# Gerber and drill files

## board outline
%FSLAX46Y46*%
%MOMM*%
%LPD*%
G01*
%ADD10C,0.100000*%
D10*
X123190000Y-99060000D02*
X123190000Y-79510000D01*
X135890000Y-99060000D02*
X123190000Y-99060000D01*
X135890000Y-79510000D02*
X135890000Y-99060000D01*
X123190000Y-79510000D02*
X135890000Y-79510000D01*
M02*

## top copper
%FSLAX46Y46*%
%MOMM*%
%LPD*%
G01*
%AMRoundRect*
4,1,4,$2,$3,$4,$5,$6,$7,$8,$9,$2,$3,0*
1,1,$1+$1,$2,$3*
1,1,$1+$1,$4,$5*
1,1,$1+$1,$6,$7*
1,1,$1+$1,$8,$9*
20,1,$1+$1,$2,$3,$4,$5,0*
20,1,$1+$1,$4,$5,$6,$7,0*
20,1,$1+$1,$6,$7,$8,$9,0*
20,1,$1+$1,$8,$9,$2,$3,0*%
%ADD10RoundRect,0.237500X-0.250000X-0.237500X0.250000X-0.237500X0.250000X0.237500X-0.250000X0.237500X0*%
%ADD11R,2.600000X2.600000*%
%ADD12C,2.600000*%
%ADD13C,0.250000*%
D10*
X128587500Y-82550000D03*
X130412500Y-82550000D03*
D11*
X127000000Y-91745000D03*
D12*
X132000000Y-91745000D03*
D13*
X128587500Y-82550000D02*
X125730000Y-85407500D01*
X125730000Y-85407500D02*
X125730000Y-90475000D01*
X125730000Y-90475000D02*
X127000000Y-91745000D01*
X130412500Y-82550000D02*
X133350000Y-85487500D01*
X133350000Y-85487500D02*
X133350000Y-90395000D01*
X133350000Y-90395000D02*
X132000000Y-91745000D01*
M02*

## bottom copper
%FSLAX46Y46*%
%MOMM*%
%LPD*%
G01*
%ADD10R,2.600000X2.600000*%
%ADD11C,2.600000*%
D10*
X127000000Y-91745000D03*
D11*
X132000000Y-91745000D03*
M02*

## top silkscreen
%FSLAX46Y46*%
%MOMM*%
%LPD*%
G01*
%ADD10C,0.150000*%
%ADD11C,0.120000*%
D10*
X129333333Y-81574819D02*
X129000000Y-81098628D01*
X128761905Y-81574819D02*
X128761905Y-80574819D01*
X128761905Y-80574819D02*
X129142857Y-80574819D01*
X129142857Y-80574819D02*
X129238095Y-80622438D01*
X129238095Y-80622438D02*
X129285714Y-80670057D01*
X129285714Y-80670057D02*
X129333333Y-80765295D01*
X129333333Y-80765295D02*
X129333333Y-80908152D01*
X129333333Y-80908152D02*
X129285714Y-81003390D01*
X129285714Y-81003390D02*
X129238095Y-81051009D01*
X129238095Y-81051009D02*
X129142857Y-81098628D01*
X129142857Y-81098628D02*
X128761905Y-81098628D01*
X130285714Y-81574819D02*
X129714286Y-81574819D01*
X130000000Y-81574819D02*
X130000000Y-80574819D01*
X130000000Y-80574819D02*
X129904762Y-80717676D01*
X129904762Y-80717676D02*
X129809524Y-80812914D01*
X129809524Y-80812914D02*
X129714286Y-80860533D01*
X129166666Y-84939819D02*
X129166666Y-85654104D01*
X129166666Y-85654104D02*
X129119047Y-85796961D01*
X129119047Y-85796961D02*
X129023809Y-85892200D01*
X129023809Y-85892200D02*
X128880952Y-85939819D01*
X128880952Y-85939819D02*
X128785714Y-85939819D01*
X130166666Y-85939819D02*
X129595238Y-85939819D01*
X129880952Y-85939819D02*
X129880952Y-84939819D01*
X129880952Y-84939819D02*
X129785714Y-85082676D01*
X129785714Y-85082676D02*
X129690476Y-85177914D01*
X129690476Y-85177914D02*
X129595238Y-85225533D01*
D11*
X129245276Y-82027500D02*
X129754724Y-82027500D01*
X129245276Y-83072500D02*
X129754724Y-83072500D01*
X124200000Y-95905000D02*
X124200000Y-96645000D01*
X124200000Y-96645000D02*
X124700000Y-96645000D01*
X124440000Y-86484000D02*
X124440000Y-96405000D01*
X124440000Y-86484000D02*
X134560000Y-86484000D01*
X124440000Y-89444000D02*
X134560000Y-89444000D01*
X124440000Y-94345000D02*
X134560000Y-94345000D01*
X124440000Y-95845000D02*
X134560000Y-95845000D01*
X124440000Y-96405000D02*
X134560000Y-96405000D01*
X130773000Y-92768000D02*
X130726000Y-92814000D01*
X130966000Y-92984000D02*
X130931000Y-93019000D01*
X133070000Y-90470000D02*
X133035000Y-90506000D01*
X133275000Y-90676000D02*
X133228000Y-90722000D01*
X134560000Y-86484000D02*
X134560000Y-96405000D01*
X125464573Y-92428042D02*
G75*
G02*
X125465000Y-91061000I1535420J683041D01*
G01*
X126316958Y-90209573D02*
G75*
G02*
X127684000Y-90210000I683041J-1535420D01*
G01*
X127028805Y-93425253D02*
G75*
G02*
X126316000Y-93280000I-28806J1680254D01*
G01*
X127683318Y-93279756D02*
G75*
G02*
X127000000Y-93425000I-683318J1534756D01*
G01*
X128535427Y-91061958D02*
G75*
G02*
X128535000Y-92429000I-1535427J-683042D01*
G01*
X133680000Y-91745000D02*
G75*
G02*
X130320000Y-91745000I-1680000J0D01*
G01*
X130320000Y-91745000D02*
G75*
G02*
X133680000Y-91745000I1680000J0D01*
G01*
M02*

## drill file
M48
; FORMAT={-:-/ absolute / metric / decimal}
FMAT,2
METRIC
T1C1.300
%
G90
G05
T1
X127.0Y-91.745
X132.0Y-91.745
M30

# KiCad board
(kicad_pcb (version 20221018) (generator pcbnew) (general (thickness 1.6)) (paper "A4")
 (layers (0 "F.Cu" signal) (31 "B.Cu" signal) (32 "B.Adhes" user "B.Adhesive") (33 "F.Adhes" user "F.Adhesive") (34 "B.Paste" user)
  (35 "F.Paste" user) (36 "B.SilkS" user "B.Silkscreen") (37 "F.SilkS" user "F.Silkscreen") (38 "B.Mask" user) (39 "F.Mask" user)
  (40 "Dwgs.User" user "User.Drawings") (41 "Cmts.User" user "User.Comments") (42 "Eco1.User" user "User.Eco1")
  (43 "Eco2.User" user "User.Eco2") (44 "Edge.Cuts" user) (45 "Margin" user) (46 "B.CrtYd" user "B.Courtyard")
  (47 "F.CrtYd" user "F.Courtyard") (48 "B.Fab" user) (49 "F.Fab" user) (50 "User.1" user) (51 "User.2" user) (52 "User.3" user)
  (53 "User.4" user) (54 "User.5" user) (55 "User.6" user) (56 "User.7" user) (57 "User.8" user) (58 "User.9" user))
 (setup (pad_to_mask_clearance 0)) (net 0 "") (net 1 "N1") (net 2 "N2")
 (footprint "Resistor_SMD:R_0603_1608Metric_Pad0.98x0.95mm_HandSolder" (layer "F.Cu") (at 129.5 82.55)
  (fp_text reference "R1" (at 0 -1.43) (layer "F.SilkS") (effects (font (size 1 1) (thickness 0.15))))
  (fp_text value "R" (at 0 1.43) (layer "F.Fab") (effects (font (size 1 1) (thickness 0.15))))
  (fp_line (start -0.254724 -0.5225) (end 0.254724 -0.5225) (stroke (width 0.12) (type solid)) (layer "F.SilkS"))
  (fp_line (start -0.254724 0.5225) (end 0.254724 0.5225) (stroke (width 0.12) (type solid)) (layer "F.SilkS"))
  (pad "1" smd roundrect (at -0.9125 0) (size 0.975 0.95) (layers "F.Cu" "F.Paste" "F.Mask") (roundrect_rratio 0.25) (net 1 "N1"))
  (pad "2" smd roundrect (at 0.9125 0) (size 0.975 0.95) (layers "F.Cu" "F.Paste" "F.Mask") (roundrect_rratio 0.25) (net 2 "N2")))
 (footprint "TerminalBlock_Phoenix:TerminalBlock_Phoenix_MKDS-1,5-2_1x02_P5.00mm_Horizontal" (layer "F.Cu") (at 127 91.745)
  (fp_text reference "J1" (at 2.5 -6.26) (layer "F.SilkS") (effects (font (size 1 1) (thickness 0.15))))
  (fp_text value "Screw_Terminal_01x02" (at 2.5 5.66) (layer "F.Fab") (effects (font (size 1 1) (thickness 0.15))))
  (fp_line (start -2.8 4.16) (end -2.8 4.9) (stroke (width 0.12) (type solid)) (layer "F.SilkS"))
  (fp_line (start -2.8 4.9) (end -2.3 4.9) (stroke (width 0.12) (type solid)) (layer "F.SilkS"))
  (fp_line (start -2.56 -5.261) (end -2.56 4.66) (stroke (width 0.12) (type solid)) (layer "F.SilkS"))
  (fp_line (start -2.56 -5.261) (end 7.56 -5.261) (stroke (width 0.12) (type solid)) (layer "F.SilkS"))
  (fp_line (start -2.56 -2.301) (end 7.56 -2.301) (stroke (width 0.12) (type solid)) (layer "F.SilkS"))
  (fp_line (start -2.56 2.6) (end 7.56 2.6) (stroke (width 0.12) (type solid)) (layer "F.SilkS"))
  (fp_line (start -2.56 4.1) (end 7.56 4.1) (stroke (width 0.12) (type solid)) (layer "F.SilkS"))
  (fp_line (start -2.56 4.66) (end 7.56 4.66) (stroke (width 0.12) (type solid)) (layer "F.SilkS"))
  (fp_line (start 3.773 1.023) (end 3.726 1.069) (stroke (width 0.12) (type solid)) (layer "F.SilkS"))
  (fp_line (start 3.966 1.239) (end 3.931 1.274) (stroke (width 0.12) (type solid)) (layer "F.SilkS"))
  (fp_line (start 6.07 -1.275) (end 6.035 -1.239) (stroke (width 0.12) (type solid)) (layer "F.SilkS"))
  (fp_line (start 6.275 -1.069) (end 6.228 -1.023) (stroke (width 0.12) (type solid)) (layer "F.SilkS"))
  (fp_line (start 7.56 -5.261) (end 7.56 4.66) (stroke (width 0.12) (type solid)) (layer "F.SilkS"))
  (fp_arc (start -1.535427 0.683042) (mid -1.680501 -0.000524) (end -1.535 -0.684) (stroke (width 0.12) (type solid)) (layer "F.SilkS"))
  (fp_arc (start -0.683042 -1.535427) (mid 0.000524 -1.680501) (end 0.684 -1.535) (stroke (width 0.12) (type solid)) (layer "F.SilkS"))
  (fp_arc (start 0.028805 1.680253) (mid -0.335551 1.646659) (end -0.684 1.535) (stroke (width 0.12) (type solid)) (layer "F.SilkS"))
  (fp_arc (start 0.683318 1.534756) (mid 0.349292 1.643288) (end 0 1.68) (stroke (width 0.12) (type solid)) (layer "F.SilkS"))
  (fp_arc (start 1.535427 -0.683042) (mid 1.680501 0.000524) (end 1.535 0.684) (stroke (width 0.12) (type solid)) (layer "F.SilkS"))
  (fp_circle (center 5 0) (end 6.68 0) (stroke (width 0.12) (type solid)) (fill none) (layer "F.SilkS"))
  (pad "1" thru_hole rect (at 0 0) (size 2.6 2.6) (drill 1.3) (layers "*.Cu" "*.Mask") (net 1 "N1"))
  (pad "2" thru_hole circle (at 5 0) (size 2.6 2.6) (drill 1.3) (layers "*.Cu" "*.Mask") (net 2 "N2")))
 (gr_line (start 123.19 99.06) (end 123.19 79.51) (stroke (width 0.1) (type solid)) (layer "Edge.Cuts"))
 (gr_line (start 135.89 99.06) (end 123.19 99.06) (stroke (width 0.1) (type solid)) (layer "Edge.Cuts"))
 (gr_line (start 135.89 79.51) (end 135.89 99.06) (stroke (width 0.1) (type solid)) (layer "Edge.Cuts"))
 (gr_line (start 123.19 79.51) (end 135.89 79.51) (stroke (width 0.1) (type solid)) (layer "Edge.Cuts"))
 (segment (start 128.5875 82.55) (end 125.73 85.4075) (width 0.25) (layer "F.Cu") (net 1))
 (segment (start 125.73 85.4075) (end 125.73 90.475) (width 0.25) (layer "F.Cu") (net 1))
 (segment (start 125.73 90.475) (end 127 91.745) (width 0.25) (layer "F.Cu") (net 1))
 (segment (start 130.4125 82.55) (end 133.35 85.4875) (width 0.25) (layer "F.Cu") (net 2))
 (segment (start 133.35 85.4875) (end 133.35 90.395) (width 0.25) (layer "F.Cu") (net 2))
 (segment (start 133.35 90.395) (end 132 91.745) (width 0.25) (layer "F.Cu") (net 2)))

